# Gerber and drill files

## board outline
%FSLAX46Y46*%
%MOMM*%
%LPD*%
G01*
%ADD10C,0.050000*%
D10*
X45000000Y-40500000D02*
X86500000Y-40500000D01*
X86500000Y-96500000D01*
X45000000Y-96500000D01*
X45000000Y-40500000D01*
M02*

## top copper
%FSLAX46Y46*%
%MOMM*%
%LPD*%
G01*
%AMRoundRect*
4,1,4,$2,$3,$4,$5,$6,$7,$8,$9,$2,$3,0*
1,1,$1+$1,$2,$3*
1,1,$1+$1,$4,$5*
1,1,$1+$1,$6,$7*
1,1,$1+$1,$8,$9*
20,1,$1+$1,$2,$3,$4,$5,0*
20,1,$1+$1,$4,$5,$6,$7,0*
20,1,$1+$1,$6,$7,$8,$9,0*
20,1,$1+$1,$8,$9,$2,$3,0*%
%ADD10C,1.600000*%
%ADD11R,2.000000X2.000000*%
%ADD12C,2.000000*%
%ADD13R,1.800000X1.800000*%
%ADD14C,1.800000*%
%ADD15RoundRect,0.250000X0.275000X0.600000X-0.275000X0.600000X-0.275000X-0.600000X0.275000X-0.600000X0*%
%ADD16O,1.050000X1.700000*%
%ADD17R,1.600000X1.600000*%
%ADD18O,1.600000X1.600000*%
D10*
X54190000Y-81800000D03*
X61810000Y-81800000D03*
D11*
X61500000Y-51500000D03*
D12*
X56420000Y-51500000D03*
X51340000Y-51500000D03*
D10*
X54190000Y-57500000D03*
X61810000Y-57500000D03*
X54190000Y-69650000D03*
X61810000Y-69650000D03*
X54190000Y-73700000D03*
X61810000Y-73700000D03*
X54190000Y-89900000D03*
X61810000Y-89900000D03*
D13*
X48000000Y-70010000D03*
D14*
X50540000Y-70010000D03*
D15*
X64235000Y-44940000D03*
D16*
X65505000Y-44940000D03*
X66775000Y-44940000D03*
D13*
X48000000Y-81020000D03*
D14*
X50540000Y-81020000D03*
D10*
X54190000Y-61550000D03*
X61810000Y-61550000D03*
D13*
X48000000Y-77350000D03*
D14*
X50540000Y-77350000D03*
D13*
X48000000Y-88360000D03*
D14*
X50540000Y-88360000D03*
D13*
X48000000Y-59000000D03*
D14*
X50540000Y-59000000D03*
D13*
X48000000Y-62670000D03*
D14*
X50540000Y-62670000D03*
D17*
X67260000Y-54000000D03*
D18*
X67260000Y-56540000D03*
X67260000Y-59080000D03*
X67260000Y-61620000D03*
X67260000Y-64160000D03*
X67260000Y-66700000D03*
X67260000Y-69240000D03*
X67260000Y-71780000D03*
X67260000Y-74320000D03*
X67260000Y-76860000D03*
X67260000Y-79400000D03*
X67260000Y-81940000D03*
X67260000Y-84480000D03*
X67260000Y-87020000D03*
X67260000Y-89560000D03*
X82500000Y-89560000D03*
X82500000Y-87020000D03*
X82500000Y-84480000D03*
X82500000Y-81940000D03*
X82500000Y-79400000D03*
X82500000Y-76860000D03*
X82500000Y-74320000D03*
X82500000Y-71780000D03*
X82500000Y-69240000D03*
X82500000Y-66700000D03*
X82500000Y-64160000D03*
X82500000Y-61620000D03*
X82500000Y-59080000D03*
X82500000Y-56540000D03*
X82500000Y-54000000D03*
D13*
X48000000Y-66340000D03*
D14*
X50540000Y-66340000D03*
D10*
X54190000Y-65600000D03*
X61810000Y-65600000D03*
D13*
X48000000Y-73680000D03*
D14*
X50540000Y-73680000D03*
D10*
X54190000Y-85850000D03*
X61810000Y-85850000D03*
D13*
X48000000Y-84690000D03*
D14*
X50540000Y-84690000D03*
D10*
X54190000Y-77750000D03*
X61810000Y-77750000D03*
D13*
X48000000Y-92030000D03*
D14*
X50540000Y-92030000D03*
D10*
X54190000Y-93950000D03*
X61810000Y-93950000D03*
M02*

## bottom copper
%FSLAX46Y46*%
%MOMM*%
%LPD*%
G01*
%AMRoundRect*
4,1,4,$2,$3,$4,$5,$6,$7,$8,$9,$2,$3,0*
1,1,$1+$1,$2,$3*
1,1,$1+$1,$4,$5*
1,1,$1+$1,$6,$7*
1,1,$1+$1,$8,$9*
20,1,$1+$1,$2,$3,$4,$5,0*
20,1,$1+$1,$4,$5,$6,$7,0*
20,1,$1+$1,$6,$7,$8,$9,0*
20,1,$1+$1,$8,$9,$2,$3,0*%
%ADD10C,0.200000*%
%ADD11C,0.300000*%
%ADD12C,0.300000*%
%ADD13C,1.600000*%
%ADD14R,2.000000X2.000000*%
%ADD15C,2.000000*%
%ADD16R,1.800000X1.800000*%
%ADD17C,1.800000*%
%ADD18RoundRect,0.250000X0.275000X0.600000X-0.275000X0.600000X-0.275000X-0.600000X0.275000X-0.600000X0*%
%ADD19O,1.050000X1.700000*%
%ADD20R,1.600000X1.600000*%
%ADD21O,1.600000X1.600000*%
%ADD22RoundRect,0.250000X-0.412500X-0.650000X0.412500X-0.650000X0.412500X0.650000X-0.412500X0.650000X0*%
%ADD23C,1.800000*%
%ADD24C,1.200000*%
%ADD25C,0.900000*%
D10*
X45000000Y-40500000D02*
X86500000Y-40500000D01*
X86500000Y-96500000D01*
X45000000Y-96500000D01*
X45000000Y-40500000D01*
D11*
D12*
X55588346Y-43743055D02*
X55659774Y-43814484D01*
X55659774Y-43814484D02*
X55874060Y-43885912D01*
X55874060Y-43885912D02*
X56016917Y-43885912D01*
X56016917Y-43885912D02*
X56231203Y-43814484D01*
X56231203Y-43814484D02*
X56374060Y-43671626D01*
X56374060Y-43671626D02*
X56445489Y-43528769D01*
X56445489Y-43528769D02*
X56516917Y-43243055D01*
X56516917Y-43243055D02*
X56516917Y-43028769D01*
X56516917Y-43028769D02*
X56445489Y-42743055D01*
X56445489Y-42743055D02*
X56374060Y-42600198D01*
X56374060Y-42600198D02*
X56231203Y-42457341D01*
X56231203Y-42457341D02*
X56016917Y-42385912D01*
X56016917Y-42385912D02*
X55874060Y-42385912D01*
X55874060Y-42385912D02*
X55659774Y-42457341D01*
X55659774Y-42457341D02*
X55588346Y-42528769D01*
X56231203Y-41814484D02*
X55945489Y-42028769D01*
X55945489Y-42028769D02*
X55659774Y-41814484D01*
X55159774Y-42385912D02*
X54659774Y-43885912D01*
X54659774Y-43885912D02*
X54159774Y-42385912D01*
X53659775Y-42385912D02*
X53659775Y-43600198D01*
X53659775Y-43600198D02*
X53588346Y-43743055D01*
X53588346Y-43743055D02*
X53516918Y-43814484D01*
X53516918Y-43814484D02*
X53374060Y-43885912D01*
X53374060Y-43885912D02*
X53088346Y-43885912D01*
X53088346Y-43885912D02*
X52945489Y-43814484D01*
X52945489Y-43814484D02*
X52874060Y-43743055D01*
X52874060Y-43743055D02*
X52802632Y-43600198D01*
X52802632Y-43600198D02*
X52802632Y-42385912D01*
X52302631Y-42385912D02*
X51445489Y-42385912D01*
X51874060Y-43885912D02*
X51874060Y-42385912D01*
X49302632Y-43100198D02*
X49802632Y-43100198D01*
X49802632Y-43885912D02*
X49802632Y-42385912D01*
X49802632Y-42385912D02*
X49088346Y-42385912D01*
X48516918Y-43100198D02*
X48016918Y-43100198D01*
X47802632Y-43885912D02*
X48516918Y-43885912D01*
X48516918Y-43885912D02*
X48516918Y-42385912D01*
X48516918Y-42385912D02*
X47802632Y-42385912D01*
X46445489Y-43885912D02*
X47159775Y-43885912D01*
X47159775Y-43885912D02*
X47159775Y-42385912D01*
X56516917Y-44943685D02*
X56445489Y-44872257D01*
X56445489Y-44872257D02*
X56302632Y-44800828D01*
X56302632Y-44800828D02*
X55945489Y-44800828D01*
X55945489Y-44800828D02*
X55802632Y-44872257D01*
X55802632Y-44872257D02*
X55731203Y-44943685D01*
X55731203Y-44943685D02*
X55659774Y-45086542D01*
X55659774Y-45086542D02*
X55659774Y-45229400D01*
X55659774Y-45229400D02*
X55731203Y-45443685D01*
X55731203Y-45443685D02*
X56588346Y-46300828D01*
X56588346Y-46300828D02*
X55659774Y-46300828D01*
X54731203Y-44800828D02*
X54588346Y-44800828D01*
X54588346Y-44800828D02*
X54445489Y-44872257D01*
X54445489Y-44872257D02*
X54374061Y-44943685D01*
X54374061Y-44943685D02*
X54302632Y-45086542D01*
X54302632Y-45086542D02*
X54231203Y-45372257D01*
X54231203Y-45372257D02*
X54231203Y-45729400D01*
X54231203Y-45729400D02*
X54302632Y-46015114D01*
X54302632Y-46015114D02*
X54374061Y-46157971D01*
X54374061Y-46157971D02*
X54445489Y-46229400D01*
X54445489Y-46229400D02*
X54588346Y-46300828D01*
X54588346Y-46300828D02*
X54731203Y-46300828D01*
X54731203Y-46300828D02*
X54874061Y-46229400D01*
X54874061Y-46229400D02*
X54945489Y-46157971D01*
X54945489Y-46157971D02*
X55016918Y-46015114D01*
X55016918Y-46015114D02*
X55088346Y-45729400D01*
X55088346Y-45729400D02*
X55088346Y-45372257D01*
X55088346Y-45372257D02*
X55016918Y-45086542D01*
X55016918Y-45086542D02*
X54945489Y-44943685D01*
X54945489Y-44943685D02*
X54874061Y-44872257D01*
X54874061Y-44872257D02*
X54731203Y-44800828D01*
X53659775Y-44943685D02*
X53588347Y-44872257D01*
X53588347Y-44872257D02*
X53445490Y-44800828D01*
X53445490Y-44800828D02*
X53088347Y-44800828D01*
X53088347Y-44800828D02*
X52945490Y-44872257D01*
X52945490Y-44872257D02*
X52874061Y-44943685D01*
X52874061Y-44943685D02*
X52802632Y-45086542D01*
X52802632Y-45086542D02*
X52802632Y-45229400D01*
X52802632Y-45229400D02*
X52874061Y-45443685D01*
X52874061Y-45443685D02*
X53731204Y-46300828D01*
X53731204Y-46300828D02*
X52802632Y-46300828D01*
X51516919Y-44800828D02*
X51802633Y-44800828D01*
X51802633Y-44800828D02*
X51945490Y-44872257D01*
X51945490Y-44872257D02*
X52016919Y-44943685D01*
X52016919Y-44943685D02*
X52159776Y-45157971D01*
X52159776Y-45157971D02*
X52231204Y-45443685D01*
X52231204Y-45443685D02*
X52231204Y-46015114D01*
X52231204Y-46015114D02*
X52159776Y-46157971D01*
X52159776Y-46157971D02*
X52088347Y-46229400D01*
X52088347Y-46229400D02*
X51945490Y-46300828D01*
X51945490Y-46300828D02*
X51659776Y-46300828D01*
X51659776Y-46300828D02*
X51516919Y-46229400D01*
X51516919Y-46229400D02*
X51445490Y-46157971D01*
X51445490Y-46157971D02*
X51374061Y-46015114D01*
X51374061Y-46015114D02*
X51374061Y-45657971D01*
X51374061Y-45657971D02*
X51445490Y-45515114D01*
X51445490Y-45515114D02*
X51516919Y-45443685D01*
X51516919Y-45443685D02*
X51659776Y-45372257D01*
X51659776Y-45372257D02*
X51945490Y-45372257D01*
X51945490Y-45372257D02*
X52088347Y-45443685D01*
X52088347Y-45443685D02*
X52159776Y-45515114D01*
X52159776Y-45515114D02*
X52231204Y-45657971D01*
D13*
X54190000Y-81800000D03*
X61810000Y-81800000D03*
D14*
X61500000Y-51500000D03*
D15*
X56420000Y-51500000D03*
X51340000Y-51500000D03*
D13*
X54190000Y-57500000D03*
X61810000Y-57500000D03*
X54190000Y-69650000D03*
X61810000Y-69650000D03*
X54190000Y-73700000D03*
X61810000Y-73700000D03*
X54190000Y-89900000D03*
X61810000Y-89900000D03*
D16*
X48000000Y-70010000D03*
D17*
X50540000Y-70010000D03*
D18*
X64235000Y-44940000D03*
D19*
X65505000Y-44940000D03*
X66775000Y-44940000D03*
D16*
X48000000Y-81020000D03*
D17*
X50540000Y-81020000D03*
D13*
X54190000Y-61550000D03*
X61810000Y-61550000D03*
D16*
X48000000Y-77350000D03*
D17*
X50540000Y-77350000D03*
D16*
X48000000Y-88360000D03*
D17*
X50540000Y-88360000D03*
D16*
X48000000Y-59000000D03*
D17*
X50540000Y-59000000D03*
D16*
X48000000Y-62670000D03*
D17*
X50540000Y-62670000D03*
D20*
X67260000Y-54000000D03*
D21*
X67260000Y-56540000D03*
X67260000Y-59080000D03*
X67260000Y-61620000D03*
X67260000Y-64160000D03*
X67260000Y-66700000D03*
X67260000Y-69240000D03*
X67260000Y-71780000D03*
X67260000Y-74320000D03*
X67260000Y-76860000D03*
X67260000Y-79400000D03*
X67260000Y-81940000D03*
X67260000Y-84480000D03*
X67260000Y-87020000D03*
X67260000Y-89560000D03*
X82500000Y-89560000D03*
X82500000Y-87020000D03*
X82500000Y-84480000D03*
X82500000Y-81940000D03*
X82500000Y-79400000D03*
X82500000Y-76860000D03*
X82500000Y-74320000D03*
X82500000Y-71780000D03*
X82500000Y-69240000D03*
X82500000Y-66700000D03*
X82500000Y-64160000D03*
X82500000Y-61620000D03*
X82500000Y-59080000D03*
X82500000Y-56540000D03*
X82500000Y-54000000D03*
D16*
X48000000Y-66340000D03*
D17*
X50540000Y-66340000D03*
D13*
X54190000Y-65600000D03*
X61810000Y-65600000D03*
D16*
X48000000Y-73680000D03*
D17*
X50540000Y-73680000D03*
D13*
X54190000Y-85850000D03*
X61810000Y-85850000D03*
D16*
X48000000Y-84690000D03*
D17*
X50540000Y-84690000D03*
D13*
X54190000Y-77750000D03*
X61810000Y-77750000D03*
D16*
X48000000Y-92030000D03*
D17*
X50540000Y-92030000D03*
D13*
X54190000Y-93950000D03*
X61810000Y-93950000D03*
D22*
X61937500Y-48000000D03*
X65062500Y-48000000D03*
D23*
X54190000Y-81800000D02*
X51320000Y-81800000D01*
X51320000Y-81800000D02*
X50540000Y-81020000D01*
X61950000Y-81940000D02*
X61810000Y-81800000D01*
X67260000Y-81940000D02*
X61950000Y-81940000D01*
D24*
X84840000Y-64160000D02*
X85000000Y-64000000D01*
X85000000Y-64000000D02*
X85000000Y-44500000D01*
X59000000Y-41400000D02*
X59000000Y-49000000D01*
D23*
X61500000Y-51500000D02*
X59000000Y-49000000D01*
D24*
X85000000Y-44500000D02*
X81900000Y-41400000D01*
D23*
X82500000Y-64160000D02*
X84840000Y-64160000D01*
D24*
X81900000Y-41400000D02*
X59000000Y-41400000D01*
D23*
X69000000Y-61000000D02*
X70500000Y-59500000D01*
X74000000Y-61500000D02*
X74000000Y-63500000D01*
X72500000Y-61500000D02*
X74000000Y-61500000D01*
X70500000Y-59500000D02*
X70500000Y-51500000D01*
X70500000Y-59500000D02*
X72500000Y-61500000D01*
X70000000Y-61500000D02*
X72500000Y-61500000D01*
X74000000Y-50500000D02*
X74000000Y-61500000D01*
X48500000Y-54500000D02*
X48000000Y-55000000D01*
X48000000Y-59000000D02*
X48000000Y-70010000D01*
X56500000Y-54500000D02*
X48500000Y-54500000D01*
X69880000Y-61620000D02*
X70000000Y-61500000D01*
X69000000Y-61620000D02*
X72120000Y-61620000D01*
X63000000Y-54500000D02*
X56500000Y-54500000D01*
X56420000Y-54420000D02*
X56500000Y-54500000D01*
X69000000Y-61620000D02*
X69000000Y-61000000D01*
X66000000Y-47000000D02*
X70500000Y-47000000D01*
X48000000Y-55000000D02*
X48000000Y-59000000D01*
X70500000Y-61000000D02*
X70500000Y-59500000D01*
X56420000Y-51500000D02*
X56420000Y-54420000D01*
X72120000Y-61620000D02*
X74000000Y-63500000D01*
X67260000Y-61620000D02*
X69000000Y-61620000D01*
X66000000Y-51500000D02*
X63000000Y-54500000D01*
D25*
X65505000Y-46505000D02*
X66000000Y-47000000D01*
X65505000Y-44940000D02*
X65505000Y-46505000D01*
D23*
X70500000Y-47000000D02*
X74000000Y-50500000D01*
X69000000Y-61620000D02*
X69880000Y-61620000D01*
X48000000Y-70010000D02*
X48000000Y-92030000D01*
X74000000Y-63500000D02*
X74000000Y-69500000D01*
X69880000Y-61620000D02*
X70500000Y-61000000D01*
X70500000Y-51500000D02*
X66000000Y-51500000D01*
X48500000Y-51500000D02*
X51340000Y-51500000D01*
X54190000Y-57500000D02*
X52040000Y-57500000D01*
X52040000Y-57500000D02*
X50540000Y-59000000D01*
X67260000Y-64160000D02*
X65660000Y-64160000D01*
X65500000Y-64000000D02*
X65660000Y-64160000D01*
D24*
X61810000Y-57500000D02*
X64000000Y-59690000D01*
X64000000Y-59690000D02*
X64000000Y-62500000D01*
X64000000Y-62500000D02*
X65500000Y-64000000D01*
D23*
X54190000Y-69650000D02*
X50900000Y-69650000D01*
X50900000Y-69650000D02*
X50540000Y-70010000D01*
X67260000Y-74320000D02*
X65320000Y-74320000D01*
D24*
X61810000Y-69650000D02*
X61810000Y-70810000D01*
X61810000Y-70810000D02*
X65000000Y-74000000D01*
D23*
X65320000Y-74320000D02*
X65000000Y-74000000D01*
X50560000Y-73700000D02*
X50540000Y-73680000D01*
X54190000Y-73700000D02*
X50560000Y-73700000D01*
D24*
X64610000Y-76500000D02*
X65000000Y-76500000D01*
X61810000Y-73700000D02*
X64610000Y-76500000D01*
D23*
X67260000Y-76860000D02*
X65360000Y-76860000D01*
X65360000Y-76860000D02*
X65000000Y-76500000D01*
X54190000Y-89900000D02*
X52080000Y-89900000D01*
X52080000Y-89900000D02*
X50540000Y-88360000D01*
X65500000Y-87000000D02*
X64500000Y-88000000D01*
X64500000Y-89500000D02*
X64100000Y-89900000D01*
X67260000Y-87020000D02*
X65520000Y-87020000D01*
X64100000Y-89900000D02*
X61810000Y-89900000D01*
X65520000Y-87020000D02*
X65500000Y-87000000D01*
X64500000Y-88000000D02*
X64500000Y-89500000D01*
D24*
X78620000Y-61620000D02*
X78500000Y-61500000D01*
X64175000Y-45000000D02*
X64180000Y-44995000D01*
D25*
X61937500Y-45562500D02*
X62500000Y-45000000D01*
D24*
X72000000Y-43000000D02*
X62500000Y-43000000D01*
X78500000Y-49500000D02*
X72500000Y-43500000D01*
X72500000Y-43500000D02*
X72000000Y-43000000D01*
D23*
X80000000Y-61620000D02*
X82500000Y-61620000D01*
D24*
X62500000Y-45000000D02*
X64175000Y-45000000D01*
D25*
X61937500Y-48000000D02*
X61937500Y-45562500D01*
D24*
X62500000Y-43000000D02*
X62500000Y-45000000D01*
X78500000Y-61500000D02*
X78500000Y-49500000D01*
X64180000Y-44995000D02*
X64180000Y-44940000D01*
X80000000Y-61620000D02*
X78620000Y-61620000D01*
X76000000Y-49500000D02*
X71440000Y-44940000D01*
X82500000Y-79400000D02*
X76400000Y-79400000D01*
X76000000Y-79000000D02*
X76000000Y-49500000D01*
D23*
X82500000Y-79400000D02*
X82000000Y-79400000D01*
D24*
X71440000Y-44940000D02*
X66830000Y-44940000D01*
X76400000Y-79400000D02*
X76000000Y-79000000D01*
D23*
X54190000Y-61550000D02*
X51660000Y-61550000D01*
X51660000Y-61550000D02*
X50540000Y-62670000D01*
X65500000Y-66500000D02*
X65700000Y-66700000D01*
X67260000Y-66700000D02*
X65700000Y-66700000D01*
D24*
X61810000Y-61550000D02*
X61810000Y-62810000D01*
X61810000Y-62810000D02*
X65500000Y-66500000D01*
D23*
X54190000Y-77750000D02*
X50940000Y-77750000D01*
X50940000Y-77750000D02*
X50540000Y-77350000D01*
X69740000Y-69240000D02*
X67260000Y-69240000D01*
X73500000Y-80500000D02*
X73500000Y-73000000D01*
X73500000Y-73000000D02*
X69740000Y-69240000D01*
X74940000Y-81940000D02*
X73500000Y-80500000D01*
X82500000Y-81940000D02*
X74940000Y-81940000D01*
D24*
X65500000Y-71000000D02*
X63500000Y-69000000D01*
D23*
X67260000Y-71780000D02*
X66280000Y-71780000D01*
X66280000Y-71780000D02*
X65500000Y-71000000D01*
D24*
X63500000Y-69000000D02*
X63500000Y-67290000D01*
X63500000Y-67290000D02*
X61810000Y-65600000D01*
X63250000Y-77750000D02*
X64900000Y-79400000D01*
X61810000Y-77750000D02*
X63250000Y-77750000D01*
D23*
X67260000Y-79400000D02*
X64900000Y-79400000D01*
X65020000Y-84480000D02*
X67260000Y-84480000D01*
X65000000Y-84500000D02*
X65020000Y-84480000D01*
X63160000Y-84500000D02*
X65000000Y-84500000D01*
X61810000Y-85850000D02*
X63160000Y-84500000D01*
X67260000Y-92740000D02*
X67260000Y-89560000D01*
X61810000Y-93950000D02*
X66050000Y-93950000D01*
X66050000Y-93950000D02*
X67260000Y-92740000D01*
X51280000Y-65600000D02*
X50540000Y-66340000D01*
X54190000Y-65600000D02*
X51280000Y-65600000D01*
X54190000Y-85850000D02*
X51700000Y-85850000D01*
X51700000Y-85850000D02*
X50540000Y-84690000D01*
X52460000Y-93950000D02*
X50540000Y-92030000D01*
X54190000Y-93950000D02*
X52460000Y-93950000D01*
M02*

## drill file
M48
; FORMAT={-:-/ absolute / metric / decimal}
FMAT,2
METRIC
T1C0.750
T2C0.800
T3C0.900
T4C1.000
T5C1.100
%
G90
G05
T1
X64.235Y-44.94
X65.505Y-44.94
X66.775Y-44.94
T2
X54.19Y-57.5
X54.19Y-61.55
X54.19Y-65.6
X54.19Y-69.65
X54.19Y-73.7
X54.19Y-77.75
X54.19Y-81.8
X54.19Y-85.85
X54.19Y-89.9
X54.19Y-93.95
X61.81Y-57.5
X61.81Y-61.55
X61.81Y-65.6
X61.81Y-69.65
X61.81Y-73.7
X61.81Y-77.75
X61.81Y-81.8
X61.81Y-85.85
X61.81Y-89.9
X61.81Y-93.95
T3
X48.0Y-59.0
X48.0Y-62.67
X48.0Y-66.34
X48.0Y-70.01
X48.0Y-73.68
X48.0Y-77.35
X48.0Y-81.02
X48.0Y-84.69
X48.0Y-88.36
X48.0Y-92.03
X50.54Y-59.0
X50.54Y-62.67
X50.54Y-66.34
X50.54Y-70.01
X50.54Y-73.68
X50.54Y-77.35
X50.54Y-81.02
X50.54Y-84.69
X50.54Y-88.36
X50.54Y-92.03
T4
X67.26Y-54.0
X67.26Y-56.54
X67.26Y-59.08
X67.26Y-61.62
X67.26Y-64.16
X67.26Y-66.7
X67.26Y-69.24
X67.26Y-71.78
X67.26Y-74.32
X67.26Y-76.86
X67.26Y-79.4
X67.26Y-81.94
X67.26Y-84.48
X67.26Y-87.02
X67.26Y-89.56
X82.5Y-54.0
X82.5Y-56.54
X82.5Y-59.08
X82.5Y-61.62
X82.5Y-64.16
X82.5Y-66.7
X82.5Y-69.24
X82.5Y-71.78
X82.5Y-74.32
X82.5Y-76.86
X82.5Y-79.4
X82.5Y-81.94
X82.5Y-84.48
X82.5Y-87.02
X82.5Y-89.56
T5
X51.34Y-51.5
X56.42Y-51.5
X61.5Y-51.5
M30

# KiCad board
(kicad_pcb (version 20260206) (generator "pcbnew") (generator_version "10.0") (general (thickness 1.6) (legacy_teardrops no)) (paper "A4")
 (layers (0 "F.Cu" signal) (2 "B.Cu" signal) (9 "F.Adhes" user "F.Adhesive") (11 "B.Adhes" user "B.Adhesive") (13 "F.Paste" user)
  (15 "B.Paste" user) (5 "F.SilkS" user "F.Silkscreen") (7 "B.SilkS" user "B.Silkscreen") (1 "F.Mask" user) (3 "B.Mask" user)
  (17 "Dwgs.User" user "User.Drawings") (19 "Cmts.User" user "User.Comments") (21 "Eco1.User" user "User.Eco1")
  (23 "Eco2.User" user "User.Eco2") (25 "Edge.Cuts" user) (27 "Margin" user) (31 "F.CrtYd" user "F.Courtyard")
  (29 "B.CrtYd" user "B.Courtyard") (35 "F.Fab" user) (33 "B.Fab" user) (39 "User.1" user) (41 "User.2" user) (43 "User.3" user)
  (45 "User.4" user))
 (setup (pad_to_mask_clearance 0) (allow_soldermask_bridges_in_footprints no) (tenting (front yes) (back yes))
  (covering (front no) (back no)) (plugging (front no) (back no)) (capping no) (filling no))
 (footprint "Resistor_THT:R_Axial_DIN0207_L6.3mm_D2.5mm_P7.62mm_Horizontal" (layer "F.Cu") (at 54.19 81.8)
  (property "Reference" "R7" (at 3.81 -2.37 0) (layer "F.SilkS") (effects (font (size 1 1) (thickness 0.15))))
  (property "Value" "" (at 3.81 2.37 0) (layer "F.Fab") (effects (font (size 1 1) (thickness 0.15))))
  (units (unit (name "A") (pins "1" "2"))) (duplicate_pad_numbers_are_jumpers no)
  (pad "1" thru_hole circle (at 0 0) (size 1.6 1.6) (drill 0.8) (layers "*.Cu" "*.Mask") (remove_unused_layers no) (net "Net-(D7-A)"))
  (pad "2" thru_hole circle (at 7.62 0) (size 1.6 1.6) (drill 0.8) (layers "*.Cu" "*.Mask") (remove_unused_layers no) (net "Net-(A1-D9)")))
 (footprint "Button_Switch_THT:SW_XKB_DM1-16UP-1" (layer "F.Cu") (at 61.5 51.5 180)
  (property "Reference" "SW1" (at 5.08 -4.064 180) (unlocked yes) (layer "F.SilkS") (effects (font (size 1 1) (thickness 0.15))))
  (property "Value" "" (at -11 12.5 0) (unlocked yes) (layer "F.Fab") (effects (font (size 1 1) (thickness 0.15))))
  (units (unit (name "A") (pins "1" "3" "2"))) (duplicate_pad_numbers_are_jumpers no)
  (pad "1" thru_hole rect (at 0 0 180) (size 2 2) (drill 1.1) (layers "*.Cu" "*.Mask") (remove_unused_layers no) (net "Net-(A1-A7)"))
  (pad "2" thru_hole circle (at 5.08 0 180) (size 2 2) (drill 1.1) (layers "*.Cu" "*.Mask") (remove_unused_layers no) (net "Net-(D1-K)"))
  (pad "3" thru_hole circle (at 10.16 0 180) (size 2 2) (drill 1.1) (layers "*.Cu" "*.Mask") (remove_unused_layers no)
   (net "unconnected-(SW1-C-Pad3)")))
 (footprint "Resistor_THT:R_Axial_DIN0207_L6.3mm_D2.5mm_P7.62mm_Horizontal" (layer "F.Cu") (at 54.19 57.5)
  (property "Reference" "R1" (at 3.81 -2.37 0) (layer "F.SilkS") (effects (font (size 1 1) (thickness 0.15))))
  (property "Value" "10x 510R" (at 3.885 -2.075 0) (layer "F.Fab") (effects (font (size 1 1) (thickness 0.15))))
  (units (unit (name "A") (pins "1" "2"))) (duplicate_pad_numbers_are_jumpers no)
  (pad "1" thru_hole circle (at 0 0) (size 1.6 1.6) (drill 0.8) (layers "*.Cu" "*.Mask") (remove_unused_layers no) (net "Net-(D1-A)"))
  (pad "2" thru_hole circle (at 7.62 0) (size 1.6 1.6) (drill 0.8) (layers "*.Cu" "*.Mask") (remove_unused_layers no) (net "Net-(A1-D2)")))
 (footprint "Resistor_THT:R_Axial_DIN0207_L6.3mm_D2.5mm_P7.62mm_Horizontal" (layer "F.Cu") (at 54.19 69.65)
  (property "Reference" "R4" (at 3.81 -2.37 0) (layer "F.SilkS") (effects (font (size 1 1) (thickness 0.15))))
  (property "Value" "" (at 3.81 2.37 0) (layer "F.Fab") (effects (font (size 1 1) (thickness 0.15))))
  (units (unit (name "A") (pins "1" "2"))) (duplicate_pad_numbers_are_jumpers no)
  (pad "1" thru_hole circle (at 0 0) (size 1.6 1.6) (drill 0.8) (layers "*.Cu" "*.Mask") (remove_unused_layers no) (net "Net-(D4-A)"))
  (pad "2" thru_hole circle (at 7.62 0) (size 1.6 1.6) (drill 0.8) (layers "*.Cu" "*.Mask") (remove_unused_layers no) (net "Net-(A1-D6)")))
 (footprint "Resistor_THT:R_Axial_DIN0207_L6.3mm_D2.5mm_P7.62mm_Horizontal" (layer "F.Cu") (at 54.19 73.7)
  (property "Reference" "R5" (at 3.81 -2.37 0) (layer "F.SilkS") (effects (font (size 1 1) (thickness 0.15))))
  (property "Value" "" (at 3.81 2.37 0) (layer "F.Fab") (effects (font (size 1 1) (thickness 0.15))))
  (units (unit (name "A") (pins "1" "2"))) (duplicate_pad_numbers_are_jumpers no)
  (pad "1" thru_hole circle (at 0 0) (size 1.6 1.6) (drill 0.8) (layers "*.Cu" "*.Mask") (remove_unused_layers no) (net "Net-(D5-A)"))
  (pad "2" thru_hole circle (at 7.62 0) (size 1.6 1.6) (drill 0.8) (layers "*.Cu" "*.Mask") (remove_unused_layers no) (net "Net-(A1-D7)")))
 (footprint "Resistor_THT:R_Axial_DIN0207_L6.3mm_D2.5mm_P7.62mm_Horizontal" (layer "F.Cu") (at 54.19 89.9)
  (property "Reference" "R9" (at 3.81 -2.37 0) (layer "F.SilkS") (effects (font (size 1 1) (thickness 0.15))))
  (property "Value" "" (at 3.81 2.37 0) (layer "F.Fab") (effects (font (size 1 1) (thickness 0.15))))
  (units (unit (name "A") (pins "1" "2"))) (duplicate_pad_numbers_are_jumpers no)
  (pad "1" thru_hole circle (at 0 0) (size 1.6 1.6) (drill 0.8) (layers "*.Cu" "*.Mask") (remove_unused_layers no) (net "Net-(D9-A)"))
  (pad "2" thru_hole circle (at 7.62 0) (size 1.6 1.6) (drill 0.8) (layers "*.Cu" "*.Mask") (remove_unused_layers no) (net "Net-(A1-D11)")))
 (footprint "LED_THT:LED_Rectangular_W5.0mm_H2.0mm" (layer "F.Cu") (at 48 70.01)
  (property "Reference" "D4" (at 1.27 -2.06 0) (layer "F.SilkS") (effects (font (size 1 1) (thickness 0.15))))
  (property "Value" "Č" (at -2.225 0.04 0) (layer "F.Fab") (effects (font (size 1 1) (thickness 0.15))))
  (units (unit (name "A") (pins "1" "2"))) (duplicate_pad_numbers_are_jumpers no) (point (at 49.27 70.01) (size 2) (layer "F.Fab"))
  (pad "1" thru_hole rect (at 0 0) (size 1.8 1.8) (drill 0.9) (layers "*.Cu" "*.Mask") (remove_unused_layers no) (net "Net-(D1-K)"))
  (pad "2" thru_hole circle (at 2.54 0) (size 1.8 1.8) (drill 0.9) (layers "*.Cu" "*.Mask") (remove_unused_layers no) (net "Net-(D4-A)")))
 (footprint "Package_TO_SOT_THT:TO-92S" (layer "F.Cu") (at 64.235 44.94)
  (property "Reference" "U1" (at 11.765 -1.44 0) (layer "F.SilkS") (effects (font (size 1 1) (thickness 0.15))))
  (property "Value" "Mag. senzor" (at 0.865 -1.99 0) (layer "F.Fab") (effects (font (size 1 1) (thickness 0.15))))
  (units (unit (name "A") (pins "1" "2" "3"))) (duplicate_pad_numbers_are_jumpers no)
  (pad "1" thru_hole roundrect (at 0 0 180) (size 1.05 1.7) (drill 0.75) (layers "*.Cu" "*.Mask") (remove_unused_layers no)
   (roundrect_rratio 0.2380952381) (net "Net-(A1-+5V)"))
  (pad "2" thru_hole oval (at 1.27 0 180) (size 1.05 1.7) (drill 0.75) (layers "*.Cu" "*.Mask") (remove_unused_layers no) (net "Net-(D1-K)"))
  (pad "3" thru_hole oval (at 2.54 0 180) (size 1.05 1.7) (drill 0.75) (layers "*.Cu" "*.Mask") (remove_unused_layers no)
   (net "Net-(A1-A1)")))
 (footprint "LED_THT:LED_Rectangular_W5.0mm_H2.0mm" (layer "F.Cu") (at 48 81.02)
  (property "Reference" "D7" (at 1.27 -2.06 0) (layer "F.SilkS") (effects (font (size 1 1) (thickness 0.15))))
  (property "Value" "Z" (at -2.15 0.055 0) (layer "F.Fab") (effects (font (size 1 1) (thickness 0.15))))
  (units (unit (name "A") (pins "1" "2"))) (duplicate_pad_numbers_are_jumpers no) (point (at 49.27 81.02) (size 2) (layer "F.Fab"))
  (pad "1" thru_hole rect (at 0 0) (size 1.8 1.8) (drill 0.9) (layers "*.Cu" "*.Mask") (remove_unused_layers no) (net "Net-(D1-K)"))
  (pad "2" thru_hole circle (at 2.54 0) (size 1.8 1.8) (drill 0.9) (layers "*.Cu" "*.Mask") (remove_unused_layers no) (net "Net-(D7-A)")))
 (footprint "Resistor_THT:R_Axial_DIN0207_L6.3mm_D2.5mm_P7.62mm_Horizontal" (layer "F.Cu") (at 54.19 61.55)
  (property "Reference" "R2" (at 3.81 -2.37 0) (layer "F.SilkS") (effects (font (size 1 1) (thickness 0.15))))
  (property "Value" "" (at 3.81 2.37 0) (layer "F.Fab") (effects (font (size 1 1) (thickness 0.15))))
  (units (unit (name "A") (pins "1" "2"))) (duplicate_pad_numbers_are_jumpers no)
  (pad "1" thru_hole circle (at 0 0) (size 1.6 1.6) (drill 0.8) (layers "*.Cu" "*.Mask") (remove_unused_layers no) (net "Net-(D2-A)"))
  (pad "2" thru_hole circle (at 7.62 0) (size 1.6 1.6) (drill 0.8) (layers "*.Cu" "*.Mask") (remove_unused_layers no) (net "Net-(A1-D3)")))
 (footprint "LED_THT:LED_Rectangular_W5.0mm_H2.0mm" (layer "F.Cu") (at 48 77.35)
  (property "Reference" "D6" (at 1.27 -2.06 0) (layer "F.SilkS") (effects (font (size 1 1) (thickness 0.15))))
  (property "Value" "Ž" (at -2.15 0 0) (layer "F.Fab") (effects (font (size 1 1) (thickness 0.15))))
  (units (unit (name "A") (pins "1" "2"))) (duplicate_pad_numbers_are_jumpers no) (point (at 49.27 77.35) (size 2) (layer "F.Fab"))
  (pad "1" thru_hole rect (at 0 0) (size 1.8 1.8) (drill 0.9) (layers "*.Cu" "*.Mask") (remove_unused_layers no) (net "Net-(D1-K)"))
  (pad "2" thru_hole circle (at 2.54 0) (size 1.8 1.8) (drill 0.9) (layers "*.Cu" "*.Mask") (remove_unused_layers no) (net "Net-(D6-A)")))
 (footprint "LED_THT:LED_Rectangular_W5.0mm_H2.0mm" (layer "F.Cu") (at 48 88.36)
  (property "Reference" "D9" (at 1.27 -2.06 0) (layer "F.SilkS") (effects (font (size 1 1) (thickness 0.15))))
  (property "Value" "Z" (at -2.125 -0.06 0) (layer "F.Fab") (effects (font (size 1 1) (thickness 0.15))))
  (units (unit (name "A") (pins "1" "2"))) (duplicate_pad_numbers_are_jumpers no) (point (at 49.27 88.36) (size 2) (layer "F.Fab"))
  (pad "1" thru_hole rect (at 0 0) (size 1.8 1.8) (drill 0.9) (layers "*.Cu" "*.Mask") (remove_unused_layers no) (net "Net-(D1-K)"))
  (pad "2" thru_hole circle (at 2.54 0) (size 1.8 1.8) (drill 0.9) (layers "*.Cu" "*.Mask") (remove_unused_layers no) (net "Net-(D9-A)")))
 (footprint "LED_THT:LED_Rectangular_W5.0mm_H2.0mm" (layer "F.Cu") (at 48 59)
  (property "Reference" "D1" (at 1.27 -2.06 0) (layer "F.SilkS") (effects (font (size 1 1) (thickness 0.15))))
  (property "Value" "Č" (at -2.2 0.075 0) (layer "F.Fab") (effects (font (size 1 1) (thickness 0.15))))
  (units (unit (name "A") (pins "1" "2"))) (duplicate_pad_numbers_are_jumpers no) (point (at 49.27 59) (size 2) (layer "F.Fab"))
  (pad "1" thru_hole rect (at 0 0) (size 1.8 1.8) (drill 0.9) (layers "*.Cu" "*.Mask") (remove_unused_layers no) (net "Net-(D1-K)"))
  (pad "2" thru_hole circle (at 2.54 0) (size 1.8 1.8) (drill 0.9) (layers "*.Cu" "*.Mask") (remove_unused_layers no) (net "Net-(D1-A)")))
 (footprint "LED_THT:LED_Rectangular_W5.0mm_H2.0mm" (layer "F.Cu") (at 48 62.67)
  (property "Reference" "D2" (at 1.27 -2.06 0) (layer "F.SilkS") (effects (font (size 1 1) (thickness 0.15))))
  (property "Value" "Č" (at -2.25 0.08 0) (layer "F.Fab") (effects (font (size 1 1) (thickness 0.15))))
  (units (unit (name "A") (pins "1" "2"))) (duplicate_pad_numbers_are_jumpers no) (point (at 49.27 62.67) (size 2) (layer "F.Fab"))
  (pad "1" thru_hole rect (at 0 0) (size 1.8 1.8) (drill 0.9) (layers "*.Cu" "*.Mask") (remove_unused_layers no) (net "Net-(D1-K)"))
  (pad "2" thru_hole circle (at 2.54 0) (size 1.8 1.8) (drill 0.9) (layers "*.Cu" "*.Mask") (remove_unused_layers no) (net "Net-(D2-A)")))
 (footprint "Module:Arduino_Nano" (layer "F.Cu") (at 67.26 54)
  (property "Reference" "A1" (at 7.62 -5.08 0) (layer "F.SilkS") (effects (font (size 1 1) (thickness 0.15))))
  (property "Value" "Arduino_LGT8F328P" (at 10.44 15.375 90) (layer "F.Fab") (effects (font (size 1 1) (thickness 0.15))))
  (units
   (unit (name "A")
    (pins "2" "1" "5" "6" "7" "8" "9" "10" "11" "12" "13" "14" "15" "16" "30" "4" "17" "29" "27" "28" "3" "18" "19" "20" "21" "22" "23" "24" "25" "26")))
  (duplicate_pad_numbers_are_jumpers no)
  (pad "1" thru_hole rect (at 0 0) (size 1.6 1.6) (drill 1) (layers "*.Cu" "*.Mask") (remove_unused_layers no)
   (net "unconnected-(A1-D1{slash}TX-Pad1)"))
  (pad "2" thru_hole oval (at 0 2.54) (size 1.6 1.6) (drill 1) (layers "*.Cu" "*.Mask") (remove_unused_layers no)
   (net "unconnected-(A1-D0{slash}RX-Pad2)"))
  (pad "3" thru_hole oval (at 0 5.08) (size 1.6 1.6) (drill 1) (layers "*.Cu" "*.Mask") (remove_unused_layers no)
   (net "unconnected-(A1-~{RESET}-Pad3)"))
  (pad "4" thru_hole oval (at 0 7.62) (size 1.6 1.6) (drill 1) (layers "*.Cu" "*.Mask") (remove_unused_layers no) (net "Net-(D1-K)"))
  (pad "5" thru_hole oval (at 0 10.16) (size 1.6 1.6) (drill 1) (layers "*.Cu" "*.Mask") (remove_unused_layers no) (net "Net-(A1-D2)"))
  (pad "6" thru_hole oval (at 0 12.7) (size 1.6 1.6) (drill 1) (layers "*.Cu" "*.Mask") (remove_unused_layers no) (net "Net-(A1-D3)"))
  (pad "7" thru_hole oval (at 0 15.24) (size 1.6 1.6) (drill 1) (layers "*.Cu" "*.Mask") (remove_unused_layers no) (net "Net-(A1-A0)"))
  (pad "8" thru_hole oval (at 0 17.78) (size 1.6 1.6) (drill 1) (layers "*.Cu" "*.Mask") (remove_unused_layers no) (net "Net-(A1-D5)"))
  (pad "9" thru_hole oval (at 0 20.32) (size 1.6 1.6) (drill 1) (layers "*.Cu" "*.Mask") (remove_unused_layers no) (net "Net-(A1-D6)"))
  (pad "10" thru_hole oval (at 0 22.86) (size 1.6 1.6) (drill 1) (layers "*.Cu" "*.Mask") (remove_unused_layers no) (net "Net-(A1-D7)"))
  (pad "11" thru_hole oval (at 0 25.4) (size 1.6 1.6) (drill 1) (layers "*.Cu" "*.Mask") (remove_unused_layers no) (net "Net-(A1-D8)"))
  (pad "12" thru_hole oval (at 0 27.94) (size 1.6 1.6) (drill 1) (layers "*.Cu" "*.Mask") (remove_unused_layers no) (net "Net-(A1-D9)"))
  (pad "13" thru_hole oval (at 0 30.48) (size 1.6 1.6) (drill 1) (layers "*.Cu" "*.Mask") (remove_unused_layers no) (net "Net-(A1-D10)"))
  (pad "14" thru_hole oval (at 0 33.02) (size 1.6 1.6) (drill 1) (layers "*.Cu" "*.Mask") (remove_unused_layers no) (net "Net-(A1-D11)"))
  (pad "15" thru_hole oval (at 0 35.56) (size 1.6 1.6) (drill 1) (layers "*.Cu" "*.Mask") (remove_unused_layers no) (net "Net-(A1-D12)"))
  (pad "16" thru_hole oval (at 15.24 35.56) (size 1.6 1.6) (drill 1) (layers "*.Cu" "*.Mask") (remove_unused_layers no)
   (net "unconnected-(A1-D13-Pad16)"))
  (pad "17" thru_hole oval (at 15.24 33.02) (size 1.6 1.6) (drill 1) (layers "*.Cu" "*.Mask") (remove_unused_layers no)
   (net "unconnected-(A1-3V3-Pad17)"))
  (pad "18" thru_hole oval (at 15.24 30.48) (size 1.6 1.6) (drill 1) (layers "*.Cu" "*.Mask") (remove_unused_layers no)
   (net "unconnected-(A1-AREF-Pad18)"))
  (pad "19" thru_hole oval (at 15.24 27.94) (size 1.6 1.6) (drill 1) (layers "*.Cu" "*.Mask") (remove_unused_layers no) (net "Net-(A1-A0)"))
  (pad "20" thru_hole oval (at 15.24 25.4) (size 1.6 1.6) (drill 1) (layers "*.Cu" "*.Mask") (remove_unused_layers no) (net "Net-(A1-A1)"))
  (pad "21" thru_hole oval (at 15.24 22.86) (size 1.6 1.6) (drill 1) (layers "*.Cu" "*.Mask") (remove_unused_layers no)
   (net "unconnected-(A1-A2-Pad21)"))
  (pad "22" thru_hole oval (at 15.24 20.32) (size 1.6 1.6) (drill 1) (layers "*.Cu" "*.Mask") (remove_unused_layers no)
   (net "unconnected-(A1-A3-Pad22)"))
  (pad "23" thru_hole oval (at 15.24 17.78) (size 1.6 1.6) (drill 1) (layers "*.Cu" "*.Mask") (remove_unused_layers no)
   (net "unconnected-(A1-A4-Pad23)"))
  (pad "24" thru_hole oval (at 15.24 15.24) (size 1.6 1.6) (drill 1) (layers "*.Cu" "*.Mask") (remove_unused_layers no)
   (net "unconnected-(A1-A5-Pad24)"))
  (pad "25" thru_hole oval (at 15.24 12.7) (size 1.6 1.6) (drill 1) (layers "*.Cu" "*.Mask") (remove_unused_layers no)
   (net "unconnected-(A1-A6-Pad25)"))
  (pad "26" thru_hole oval (at 15.24 10.16) (size 1.6 1.6) (drill 1) (layers "*.Cu" "*.Mask") (remove_unused_layers no) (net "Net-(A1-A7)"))
  (pad "27" thru_hole oval (at 15.24 7.62) (size 1.6 1.6) (drill 1) (layers "*.Cu" "*.Mask") (remove_unused_layers no) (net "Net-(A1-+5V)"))
  (pad "28" thru_hole oval (at 15.24 5.08) (size 1.6 1.6) (drill 1) (layers "*.Cu" "*.Mask") (remove_unused_layers no)
   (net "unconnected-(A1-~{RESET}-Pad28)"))
  (pad "29" thru_hole oval (at 15.24 2.54) (size 1.6 1.6) (drill 1) (layers "*.Cu" "*.Mask") (remove_unused_layers no)
   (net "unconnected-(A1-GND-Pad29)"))
  (pad "30" thru_hole oval (at 15.24 0) (size 1.6 1.6) (drill 1) (layers "*.Cu" "*.Mask") (remove_unused_layers no)
   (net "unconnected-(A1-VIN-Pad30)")))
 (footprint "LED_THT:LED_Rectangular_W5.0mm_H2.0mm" (layer "F.Cu") (at 48 66.34)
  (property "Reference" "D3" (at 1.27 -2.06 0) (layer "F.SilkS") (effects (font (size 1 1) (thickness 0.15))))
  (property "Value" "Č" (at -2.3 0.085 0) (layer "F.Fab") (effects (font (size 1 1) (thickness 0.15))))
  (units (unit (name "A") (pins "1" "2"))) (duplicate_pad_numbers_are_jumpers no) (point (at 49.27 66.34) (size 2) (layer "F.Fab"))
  (pad "1" thru_hole rect (at 0 0) (size 1.8 1.8) (drill 0.9) (layers "*.Cu" "*.Mask") (remove_unused_layers no) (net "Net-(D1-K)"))
  (pad "2" thru_hole circle (at 2.54 0) (size 1.8 1.8) (drill 0.9) (layers "*.Cu" "*.Mask") (remove_unused_layers no) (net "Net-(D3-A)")))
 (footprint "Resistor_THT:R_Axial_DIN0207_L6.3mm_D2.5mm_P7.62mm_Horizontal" (layer "F.Cu") (at 54.19 65.6)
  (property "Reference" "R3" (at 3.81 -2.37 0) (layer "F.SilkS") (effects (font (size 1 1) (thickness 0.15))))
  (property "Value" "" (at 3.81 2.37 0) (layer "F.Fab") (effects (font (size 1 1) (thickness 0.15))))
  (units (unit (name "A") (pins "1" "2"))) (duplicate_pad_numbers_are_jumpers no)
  (pad "1" thru_hole circle (at 0 0) (size 1.6 1.6) (drill 0.8) (layers "*.Cu" "*.Mask") (remove_unused_layers no) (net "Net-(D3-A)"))
  (pad "2" thru_hole circle (at 7.62 0) (size 1.6 1.6) (drill 0.8) (layers "*.Cu" "*.Mask") (remove_unused_layers no) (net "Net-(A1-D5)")))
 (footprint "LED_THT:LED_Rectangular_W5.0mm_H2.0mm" (layer "F.Cu") (at 48 73.68)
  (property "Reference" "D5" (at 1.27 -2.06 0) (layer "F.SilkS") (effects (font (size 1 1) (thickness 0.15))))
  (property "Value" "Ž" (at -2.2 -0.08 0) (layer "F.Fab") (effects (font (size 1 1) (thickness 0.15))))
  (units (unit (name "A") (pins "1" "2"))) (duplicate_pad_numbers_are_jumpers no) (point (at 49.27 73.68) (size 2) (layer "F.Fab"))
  (pad "1" thru_hole rect (at 0 0) (size 1.8 1.8) (drill 0.9) (layers "*.Cu" "*.Mask") (remove_unused_layers no) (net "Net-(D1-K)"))
  (pad "2" thru_hole circle (at 2.54 0) (size 1.8 1.8) (drill 0.9) (layers "*.Cu" "*.Mask") (remove_unused_layers no) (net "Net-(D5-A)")))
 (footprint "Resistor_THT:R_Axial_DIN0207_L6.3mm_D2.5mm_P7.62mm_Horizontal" (layer "F.Cu") (at 54.19 85.85)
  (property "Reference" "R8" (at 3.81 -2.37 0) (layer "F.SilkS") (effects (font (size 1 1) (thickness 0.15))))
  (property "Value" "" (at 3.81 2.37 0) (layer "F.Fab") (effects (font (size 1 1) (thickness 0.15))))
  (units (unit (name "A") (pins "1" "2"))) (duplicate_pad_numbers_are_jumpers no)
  (pad "1" thru_hole circle (at 0 0) (size 1.6 1.6) (drill 0.8) (layers "*.Cu" "*.Mask") (remove_unused_layers no) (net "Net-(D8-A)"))
  (pad "2" thru_hole circle (at 7.62 0) (size 1.6 1.6) (drill 0.8) (layers "*.Cu" "*.Mask") (remove_unused_layers no) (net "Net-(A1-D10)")))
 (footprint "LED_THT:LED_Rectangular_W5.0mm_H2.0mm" (layer "F.Cu") (at 48 84.69)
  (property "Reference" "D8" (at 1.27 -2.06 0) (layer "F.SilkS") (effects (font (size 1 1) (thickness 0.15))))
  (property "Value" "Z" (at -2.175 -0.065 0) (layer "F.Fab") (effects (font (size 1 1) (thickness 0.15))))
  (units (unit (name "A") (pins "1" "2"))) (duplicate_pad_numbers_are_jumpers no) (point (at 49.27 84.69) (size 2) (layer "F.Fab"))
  (pad "1" thru_hole rect (at 0 0) (size 1.8 1.8) (drill 0.9) (layers "*.Cu" "*.Mask") (remove_unused_layers no) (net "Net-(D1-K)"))
  (pad "2" thru_hole circle (at 2.54 0) (size 1.8 1.8) (drill 0.9) (layers "*.Cu" "*.Mask") (remove_unused_layers no) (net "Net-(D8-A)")))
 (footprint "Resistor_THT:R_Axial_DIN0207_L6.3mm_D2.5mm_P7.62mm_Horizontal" (layer "F.Cu") (at 54.19 77.75)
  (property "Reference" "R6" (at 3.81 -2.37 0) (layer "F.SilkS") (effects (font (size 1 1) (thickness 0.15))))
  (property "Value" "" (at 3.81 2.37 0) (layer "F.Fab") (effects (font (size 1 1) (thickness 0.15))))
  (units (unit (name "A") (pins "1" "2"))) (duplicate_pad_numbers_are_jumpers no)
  (pad "1" thru_hole circle (at 0 0) (size 1.6 1.6) (drill 0.8) (layers "*.Cu" "*.Mask") (remove_unused_layers no) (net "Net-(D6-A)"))
  (pad "2" thru_hole circle (at 7.62 0) (size 1.6 1.6) (drill 0.8) (layers "*.Cu" "*.Mask") (remove_unused_layers no) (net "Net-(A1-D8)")))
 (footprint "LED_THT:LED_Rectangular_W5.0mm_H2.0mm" (layer "F.Cu") (at 48 92.03)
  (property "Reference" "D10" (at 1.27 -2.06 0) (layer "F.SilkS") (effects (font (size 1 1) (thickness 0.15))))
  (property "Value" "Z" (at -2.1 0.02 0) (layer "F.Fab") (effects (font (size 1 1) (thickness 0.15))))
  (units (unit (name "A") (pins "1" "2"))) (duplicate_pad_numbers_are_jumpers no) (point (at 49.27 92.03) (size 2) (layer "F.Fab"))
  (pad "1" thru_hole rect (at 0 0) (size 1.8 1.8) (drill 0.9) (layers "*.Cu" "*.Mask") (remove_unused_layers no) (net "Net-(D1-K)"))
  (pad "2" thru_hole circle (at 2.54 0) (size 1.8 1.8) (drill 0.9) (layers "*.Cu" "*.Mask") (remove_unused_layers no) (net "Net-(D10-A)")))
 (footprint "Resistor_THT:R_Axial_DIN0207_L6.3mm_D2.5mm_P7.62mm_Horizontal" (layer "F.Cu") (at 54.19 93.95)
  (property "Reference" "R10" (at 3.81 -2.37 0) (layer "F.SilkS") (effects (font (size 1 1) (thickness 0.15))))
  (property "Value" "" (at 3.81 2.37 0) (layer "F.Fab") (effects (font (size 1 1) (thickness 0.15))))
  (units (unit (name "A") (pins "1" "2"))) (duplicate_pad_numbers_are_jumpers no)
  (pad "1" thru_hole circle (at 0 0) (size 1.6 1.6) (drill 0.8) (layers "*.Cu" "*.Mask") (remove_unused_layers no) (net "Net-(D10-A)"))
  (pad "2" thru_hole circle (at 7.62 0) (size 1.6 1.6) (drill 0.8) (layers "*.Cu" "*.Mask") (remove_unused_layers no) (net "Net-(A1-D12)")))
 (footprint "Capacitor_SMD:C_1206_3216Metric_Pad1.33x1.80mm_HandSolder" (layer "B.Cu") (at 63.5 48)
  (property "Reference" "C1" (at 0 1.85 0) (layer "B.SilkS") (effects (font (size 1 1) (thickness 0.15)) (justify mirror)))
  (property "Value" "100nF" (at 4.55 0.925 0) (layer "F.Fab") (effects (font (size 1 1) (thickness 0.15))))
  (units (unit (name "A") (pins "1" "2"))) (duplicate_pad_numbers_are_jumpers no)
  (pad "1" smd roundrect (at -1.5625 0) (size 1.325 1.8) (layers "B.Cu" "B.Mask" "B.Paste") (roundrect_rratio 0.188679) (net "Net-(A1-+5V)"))
  (pad "2" smd roundrect (at 1.5625 0) (size 1.325 1.8) (layers "B.Cu" "B.Mask" "B.Paste") (roundrect_rratio 0.188679) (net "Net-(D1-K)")))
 (gr_rect (start 45 40.5) (end 86.5 96.5) (stroke (width 0.2) (type default)) (fill no) (layer "B.Cu"))
 (gr_rect (start 45 40.5) (end 86.5 96.5) (stroke (width 0.05) (type default)) (fill no) (layer "Edge.Cuts"))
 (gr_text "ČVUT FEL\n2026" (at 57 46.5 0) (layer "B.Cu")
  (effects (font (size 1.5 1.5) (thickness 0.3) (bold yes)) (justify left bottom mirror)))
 (segment (start 54.19 81.8) (end 51.32 81.8) (width 1.8) (layer "B.Cu") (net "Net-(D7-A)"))
 (segment (start 51.32 81.8) (end 50.54 81.02) (width 1.8) (layer "B.Cu") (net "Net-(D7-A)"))
 (segment (start 61.95 81.94) (end 61.81 81.8) (width 1.8) (layer "B.Cu") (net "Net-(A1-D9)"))
 (segment (start 67.26 81.94) (end 61.95 81.94) (width 1.8) (layer "B.Cu") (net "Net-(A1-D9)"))
 (segment (start 84.84 64.16) (end 85 64) (width 1.2) (layer "B.Cu") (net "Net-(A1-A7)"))
 (segment (start 85 64) (end 85 44.5) (width 1.2) (layer "B.Cu") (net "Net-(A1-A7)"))
 (segment (start 59 41.4) (end 59 49) (width 1.2) (layer "B.Cu") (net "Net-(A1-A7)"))
 (segment (start 61.5 51.5) (end 59 49) (width 1.8) (layer "B.Cu") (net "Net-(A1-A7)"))
 (segment (start 85 44.5) (end 81.9 41.4) (width 1.2) (layer "B.Cu") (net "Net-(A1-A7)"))
 (segment (start 82.5 64.16) (end 84.84 64.16) (width 1.8) (layer "B.Cu") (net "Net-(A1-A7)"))
 (segment (start 81.9 41.4) (end 59 41.4) (width 1.2) (layer "B.Cu") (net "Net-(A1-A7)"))
 (segment (start 69 61) (end 70.5 59.5) (width 1.8) (layer "B.Cu") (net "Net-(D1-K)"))
 (segment (start 74 61.5) (end 74 63.5) (width 1.8) (layer "B.Cu") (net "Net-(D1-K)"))
 (segment (start 72.5 61.5) (end 74 61.5) (width 1.8) (layer "B.Cu") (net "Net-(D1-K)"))
 (segment (start 70.5 59.5) (end 70.5 51.5) (width 1.8) (layer "B.Cu") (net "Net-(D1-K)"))
 (segment (start 70.5 59.5) (end 72.5 61.5) (width 1.8) (layer "B.Cu") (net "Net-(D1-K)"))
 (segment (start 70 61.5) (end 72.5 61.5) (width 1.8) (layer "B.Cu") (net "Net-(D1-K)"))
 (segment (start 74 50.5) (end 74 61.5) (width 1.8) (layer "B.Cu") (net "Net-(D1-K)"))
 (segment (start 48.5 54.5) (end 48 55) (width 1.8) (layer "B.Cu") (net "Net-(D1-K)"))
 (segment (start 48 59) (end 48 70.01) (width 1.8) (layer "B.Cu") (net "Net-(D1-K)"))
 (segment (start 56.5 54.5) (end 48.5 54.5) (width 1.8) (layer "B.Cu") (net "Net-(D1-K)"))
 (segment (start 69.88 61.62) (end 70 61.5) (width 1.8) (layer "B.Cu") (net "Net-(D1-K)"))
 (segment (start 69 61.62) (end 72.12 61.62) (width 1.8) (layer "B.Cu") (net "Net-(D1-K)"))
 (segment (start 63 54.5) (end 56.5 54.5) (width 1.8) (layer "B.Cu") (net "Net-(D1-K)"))
 (segment (start 56.42 54.42) (end 56.5 54.5) (width 1.8) (layer "B.Cu") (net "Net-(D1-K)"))
 (segment (start 69 61.62) (end 69 61) (width 1.8) (layer "B.Cu") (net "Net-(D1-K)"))
 (segment (start 66 47) (end 70.5 47) (width 1.8) (layer "B.Cu") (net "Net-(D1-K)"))
 (segment (start 48 55) (end 48 59) (width 1.8) (layer "B.Cu") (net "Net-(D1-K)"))
 (segment (start 70.5 61) (end 70.5 59.5) (width 1.8) (layer "B.Cu") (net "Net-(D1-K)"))
 (segment (start 56.42 51.5) (end 56.42 54.42) (width 1.8) (layer "B.Cu") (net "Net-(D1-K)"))
 (segment (start 72.12 61.62) (end 74 63.5) (width 1.8) (layer "B.Cu") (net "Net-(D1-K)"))
 (segment (start 67.26 61.62) (end 69 61.62) (width 1.8) (layer "B.Cu") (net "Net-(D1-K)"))
 (segment (start 66 51.5) (end 63 54.5) (width 1.8) (layer "B.Cu") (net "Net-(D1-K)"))
 (segment (start 65.505 46.505) (end 66 47) (width 0.9) (layer "B.Cu") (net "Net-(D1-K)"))
 (segment (start 65.505 44.94) (end 65.505 46.505) (width 0.9) (layer "B.Cu") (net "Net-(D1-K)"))
 (segment (start 70.5 47) (end 74 50.5) (width 1.8) (layer "B.Cu") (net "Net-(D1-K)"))
 (segment (start 69 61.62) (end 69.88 61.62) (width 1.8) (layer "B.Cu") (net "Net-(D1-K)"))
 (segment (start 48 70.01) (end 48 92.03) (width 1.8) (layer "B.Cu") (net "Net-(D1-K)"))
 (segment (start 74 63.5) (end 74 69.5) (width 1.8) (layer "B.Cu") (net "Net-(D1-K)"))
 (segment (start 69.88 61.62) (end 70.5 61) (width 1.8) (layer "B.Cu") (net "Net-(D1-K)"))
 (segment (start 70.5 51.5) (end 66 51.5) (width 1.8) (layer "B.Cu") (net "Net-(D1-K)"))
 (segment (start 48.5 51.5) (end 51.34 51.5) (width 1.8) (layer "B.Cu") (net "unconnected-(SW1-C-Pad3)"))
 (segment (start 54.19 57.5) (end 52.04 57.5) (width 1.8) (layer "B.Cu") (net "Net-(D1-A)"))
 (segment (start 52.04 57.5) (end 50.54 59) (width 1.8) (layer "B.Cu") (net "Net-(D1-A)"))
 (segment (start 67.26 64.16) (end 65.66 64.16) (width 1.8) (layer "B.Cu") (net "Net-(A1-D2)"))
 (segment (start 65.5 64) (end 65.66 64.16) (width 1.8) (layer "B.Cu") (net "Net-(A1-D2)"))
 (segment (start 61.81 57.5) (end 64 59.69) (width 1.2) (layer "B.Cu") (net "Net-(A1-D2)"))
 (segment (start 64 59.69) (end 64 62.5) (width 1.2) (layer "B.Cu") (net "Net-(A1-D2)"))
 (segment (start 64 62.5) (end 65.5 64) (width 1.2) (layer "B.Cu") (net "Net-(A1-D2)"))
 (segment (start 54.19 69.65) (end 50.9 69.65) (width 1.8) (layer "B.Cu") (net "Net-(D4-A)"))
 (segment (start 50.9 69.65) (end 50.54 70.01) (width 1.8) (layer "B.Cu") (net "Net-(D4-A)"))
 (segment (start 67.26 74.32) (end 65.32 74.32) (width 1.8) (layer "B.Cu") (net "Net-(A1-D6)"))
 (segment (start 61.81 69.65) (end 61.81 70.81) (width 1.2) (layer "B.Cu") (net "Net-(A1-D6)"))
 (segment (start 61.81 70.81) (end 65 74) (width 1.2) (layer "B.Cu") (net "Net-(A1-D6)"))
 (segment (start 65.32 74.32) (end 65 74) (width 1.8) (layer "B.Cu") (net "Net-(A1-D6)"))
 (segment (start 50.56 73.7) (end 50.54 73.68) (width 1.8) (layer "B.Cu") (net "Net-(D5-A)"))
 (segment (start 54.19 73.7) (end 50.56 73.7) (width 1.8) (layer "B.Cu") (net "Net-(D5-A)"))
 (segment (start 64.61 76.5) (end 65 76.5) (width 1.2) (layer "B.Cu") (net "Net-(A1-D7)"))
 (segment (start 61.81 73.7) (end 64.61 76.5) (width 1.2) (layer "B.Cu") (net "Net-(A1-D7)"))
 (segment (start 67.26 76.86) (end 65.36 76.86) (width 1.8) (layer "B.Cu") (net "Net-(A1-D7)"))
 (segment (start 65.36 76.86) (end 65 76.5) (width 1.8) (layer "B.Cu") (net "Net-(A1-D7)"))
 (segment (start 54.19 89.9) (end 52.08 89.9) (width 1.8) (layer "B.Cu") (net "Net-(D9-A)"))
 (segment (start 52.08 89.9) (end 50.54 88.36) (width 1.8) (layer "B.Cu") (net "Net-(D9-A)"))
 (segment (start 65.5 87) (end 64.5 88) (width 1.8) (layer "B.Cu") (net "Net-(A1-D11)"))
 (segment (start 64.5 89.5) (end 64.1 89.9) (width 1.8) (layer "B.Cu") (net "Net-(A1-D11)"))
 (segment (start 67.26 87.02) (end 65.52 87.02) (width 1.8) (layer "B.Cu") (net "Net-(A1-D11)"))
 (segment (start 64.1 89.9) (end 61.81 89.9) (width 1.8) (layer "B.Cu") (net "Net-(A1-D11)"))
 (segment (start 65.52 87.02) (end 65.5 87) (width 1.8) (layer "B.Cu") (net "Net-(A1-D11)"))
 (segment (start 64.5 88) (end 64.5 89.5) (width 1.8) (layer "B.Cu") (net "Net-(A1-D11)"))
 (segment (start 78.62 61.62) (end 78.5 61.5) (width 1.2) (layer "B.Cu") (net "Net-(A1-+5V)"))
 (segment (start 64.175 45) (end 64.18 44.995) (width 1.2) (layer "B.Cu") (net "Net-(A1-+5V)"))
 (segment (start 61.9375 45.5625) (end 62.5 45) (width 0.9) (layer "B.Cu") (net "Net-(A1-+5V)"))
 (segment (start 72 43) (end 62.5 43) (width 1.2) (layer "B.Cu") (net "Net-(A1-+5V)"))
 (segment (start 78.5 49.5) (end 72.5 43.5) (width 1.2) (layer "B.Cu") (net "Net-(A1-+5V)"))
 (segment (start 72.5 43.5) (end 72 43) (width 1.2) (layer "B.Cu") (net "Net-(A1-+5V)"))
 (segment (start 80 61.62) (end 82.5 61.62) (width 1.8) (layer "B.Cu") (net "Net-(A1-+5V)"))
 (segment (start 62.5 45) (end 64.175 45) (width 1.2) (layer "B.Cu") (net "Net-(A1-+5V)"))
 (segment (start 61.9375 48) (end 61.9375 45.5625) (width 0.9) (layer "B.Cu") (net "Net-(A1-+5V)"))
 (segment (start 62.5 43) (end 62.5 45) (width 1.2) (layer "B.Cu") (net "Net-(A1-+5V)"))
 (segment (start 78.5 61.5) (end 78.5 49.5) (width 1.2) (layer "B.Cu") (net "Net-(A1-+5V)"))
 (segment (start 64.18 44.995) (end 64.18 44.94) (width 1.2) (layer "B.Cu") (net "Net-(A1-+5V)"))
 (segment (start 80 61.62) (end 78.62 61.62) (width 1.2) (layer "B.Cu") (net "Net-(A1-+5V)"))
 (segment (start 76 49.5) (end 71.44 44.94) (width 1.2) (layer "B.Cu") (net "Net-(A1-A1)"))
 (segment (start 82.5 79.4) (end 76.4 79.4) (width 1.2) (layer "B.Cu") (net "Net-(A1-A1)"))
 (segment (start 76 79) (end 76 49.5) (width 1.2) (layer "B.Cu") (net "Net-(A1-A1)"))
 (segment (start 82.5 79.4) (end 82 79.4) (width 1.8) (layer "B.Cu") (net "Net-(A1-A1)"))
 (segment (start 71.44 44.94) (end 66.83 44.94) (width 1.2) (layer "B.Cu") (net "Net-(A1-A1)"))
 (segment (start 76.4 79.4) (end 76 79) (width 1.2) (layer "B.Cu") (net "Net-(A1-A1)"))
 (segment (start 54.19 61.55) (end 51.66 61.55) (width 1.8) (layer "B.Cu") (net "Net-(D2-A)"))
 (segment (start 51.66 61.55) (end 50.54 62.67) (width 1.8) (layer "B.Cu") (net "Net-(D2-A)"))
 (segment (start 65.5 66.5) (end 65.7 66.7) (width 1.8) (layer "B.Cu") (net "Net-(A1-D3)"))
 (segment (start 67.26 66.7) (end 65.7 66.7) (width 1.8) (layer "B.Cu") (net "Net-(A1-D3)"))
 (segment (start 61.81 61.55) (end 61.81 62.81) (width 1.2) (layer "B.Cu") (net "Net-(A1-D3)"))
 (segment (start 61.81 62.81) (end 65.5 66.5) (width 1.2) (layer "B.Cu") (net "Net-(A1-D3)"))
 (segment (start 54.19 77.75) (end 50.94 77.75) (width 1.8) (layer "B.Cu") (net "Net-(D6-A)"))
 (segment (start 50.94 77.75) (end 50.54 77.35) (width 1.8) (layer "B.Cu") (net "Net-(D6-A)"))
 (segment (start 69.74 69.24) (end 67.26 69.24) (width 1.8) (layer "B.Cu") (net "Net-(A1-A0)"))
 (segment (start 73.5 80.5) (end 73.5 73) (width 1.8) (layer "B.Cu") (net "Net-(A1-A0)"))
 (segment (start 73.5 73) (end 69.74 69.24) (width 1.8) (layer "B.Cu") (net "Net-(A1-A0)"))
 (segment (start 74.94 81.94) (end 73.5 80.5) (width 1.8) (layer "B.Cu") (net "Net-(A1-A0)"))
 (segment (start 82.5 81.94) (end 74.94 81.94) (width 1.8) (layer "B.Cu") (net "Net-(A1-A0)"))
 (segment (start 65.5 71) (end 63.5 69) (width 1.2) (layer "B.Cu") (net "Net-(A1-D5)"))
 (segment (start 67.26 71.78) (end 66.28 71.78) (width 1.8) (layer "B.Cu") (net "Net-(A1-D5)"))
 (segment (start 66.28 71.78) (end 65.5 71) (width 1.8) (layer "B.Cu") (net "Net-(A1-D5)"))
 (segment (start 63.5 69) (end 63.5 67.29) (width 1.2) (layer "B.Cu") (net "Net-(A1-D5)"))
 (segment (start 63.5 67.29) (end 61.81 65.6) (width 1.2) (layer "B.Cu") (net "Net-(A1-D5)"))
 (segment (start 63.25 77.75) (end 64.9 79.4) (width 1.2) (layer "B.Cu") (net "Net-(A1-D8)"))
 (segment (start 61.81 77.75) (end 63.25 77.75) (width 1.2) (layer "B.Cu") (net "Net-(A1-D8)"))
 (segment (start 67.26 79.4) (end 64.9 79.4) (width 1.8) (layer "B.Cu") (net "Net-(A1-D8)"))
 (segment (start 65.02 84.48) (end 67.26 84.48) (width 1.8) (layer "B.Cu") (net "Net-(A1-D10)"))
 (segment (start 65 84.5) (end 65.02 84.48) (width 1.8) (layer "B.Cu") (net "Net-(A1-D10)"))
 (segment (start 63.16 84.5) (end 65 84.5) (width 1.8) (layer "B.Cu") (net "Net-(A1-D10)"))
 (segment (start 61.81 85.85) (end 63.16 84.5) (width 1.8) (layer "B.Cu") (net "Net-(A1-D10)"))
 (segment (start 67.26 92.74) (end 67.26 89.56) (width 1.8) (layer "B.Cu") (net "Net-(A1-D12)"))
 (segment (start 61.81 93.95) (end 66.05 93.95) (width 1.8) (layer "B.Cu") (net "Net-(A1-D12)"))
 (segment (start 66.05 93.95) (end 67.26 92.74) (width 1.8) (layer "B.Cu") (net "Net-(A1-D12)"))
 (segment (start 51.28 65.6) (end 50.54 66.34) (width 1.8) (layer "B.Cu") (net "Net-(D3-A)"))
 (segment (start 54.19 65.6) (end 51.28 65.6) (width 1.8) (layer "B.Cu") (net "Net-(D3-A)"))
 (segment (start 54.19 85.85) (end 51.7 85.85) (width 1.8) (layer "B.Cu") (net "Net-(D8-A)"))
 (segment (start 51.7 85.85) (end 50.54 84.69) (width 1.8) (layer "B.Cu") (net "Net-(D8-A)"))
 (segment (start 52.46 93.95) (end 50.54 92.03) (width 1.8) (layer "B.Cu") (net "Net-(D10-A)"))
 (segment (start 54.19 93.95) (end 52.46 93.95) (width 1.8) (layer "B.Cu") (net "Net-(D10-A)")))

